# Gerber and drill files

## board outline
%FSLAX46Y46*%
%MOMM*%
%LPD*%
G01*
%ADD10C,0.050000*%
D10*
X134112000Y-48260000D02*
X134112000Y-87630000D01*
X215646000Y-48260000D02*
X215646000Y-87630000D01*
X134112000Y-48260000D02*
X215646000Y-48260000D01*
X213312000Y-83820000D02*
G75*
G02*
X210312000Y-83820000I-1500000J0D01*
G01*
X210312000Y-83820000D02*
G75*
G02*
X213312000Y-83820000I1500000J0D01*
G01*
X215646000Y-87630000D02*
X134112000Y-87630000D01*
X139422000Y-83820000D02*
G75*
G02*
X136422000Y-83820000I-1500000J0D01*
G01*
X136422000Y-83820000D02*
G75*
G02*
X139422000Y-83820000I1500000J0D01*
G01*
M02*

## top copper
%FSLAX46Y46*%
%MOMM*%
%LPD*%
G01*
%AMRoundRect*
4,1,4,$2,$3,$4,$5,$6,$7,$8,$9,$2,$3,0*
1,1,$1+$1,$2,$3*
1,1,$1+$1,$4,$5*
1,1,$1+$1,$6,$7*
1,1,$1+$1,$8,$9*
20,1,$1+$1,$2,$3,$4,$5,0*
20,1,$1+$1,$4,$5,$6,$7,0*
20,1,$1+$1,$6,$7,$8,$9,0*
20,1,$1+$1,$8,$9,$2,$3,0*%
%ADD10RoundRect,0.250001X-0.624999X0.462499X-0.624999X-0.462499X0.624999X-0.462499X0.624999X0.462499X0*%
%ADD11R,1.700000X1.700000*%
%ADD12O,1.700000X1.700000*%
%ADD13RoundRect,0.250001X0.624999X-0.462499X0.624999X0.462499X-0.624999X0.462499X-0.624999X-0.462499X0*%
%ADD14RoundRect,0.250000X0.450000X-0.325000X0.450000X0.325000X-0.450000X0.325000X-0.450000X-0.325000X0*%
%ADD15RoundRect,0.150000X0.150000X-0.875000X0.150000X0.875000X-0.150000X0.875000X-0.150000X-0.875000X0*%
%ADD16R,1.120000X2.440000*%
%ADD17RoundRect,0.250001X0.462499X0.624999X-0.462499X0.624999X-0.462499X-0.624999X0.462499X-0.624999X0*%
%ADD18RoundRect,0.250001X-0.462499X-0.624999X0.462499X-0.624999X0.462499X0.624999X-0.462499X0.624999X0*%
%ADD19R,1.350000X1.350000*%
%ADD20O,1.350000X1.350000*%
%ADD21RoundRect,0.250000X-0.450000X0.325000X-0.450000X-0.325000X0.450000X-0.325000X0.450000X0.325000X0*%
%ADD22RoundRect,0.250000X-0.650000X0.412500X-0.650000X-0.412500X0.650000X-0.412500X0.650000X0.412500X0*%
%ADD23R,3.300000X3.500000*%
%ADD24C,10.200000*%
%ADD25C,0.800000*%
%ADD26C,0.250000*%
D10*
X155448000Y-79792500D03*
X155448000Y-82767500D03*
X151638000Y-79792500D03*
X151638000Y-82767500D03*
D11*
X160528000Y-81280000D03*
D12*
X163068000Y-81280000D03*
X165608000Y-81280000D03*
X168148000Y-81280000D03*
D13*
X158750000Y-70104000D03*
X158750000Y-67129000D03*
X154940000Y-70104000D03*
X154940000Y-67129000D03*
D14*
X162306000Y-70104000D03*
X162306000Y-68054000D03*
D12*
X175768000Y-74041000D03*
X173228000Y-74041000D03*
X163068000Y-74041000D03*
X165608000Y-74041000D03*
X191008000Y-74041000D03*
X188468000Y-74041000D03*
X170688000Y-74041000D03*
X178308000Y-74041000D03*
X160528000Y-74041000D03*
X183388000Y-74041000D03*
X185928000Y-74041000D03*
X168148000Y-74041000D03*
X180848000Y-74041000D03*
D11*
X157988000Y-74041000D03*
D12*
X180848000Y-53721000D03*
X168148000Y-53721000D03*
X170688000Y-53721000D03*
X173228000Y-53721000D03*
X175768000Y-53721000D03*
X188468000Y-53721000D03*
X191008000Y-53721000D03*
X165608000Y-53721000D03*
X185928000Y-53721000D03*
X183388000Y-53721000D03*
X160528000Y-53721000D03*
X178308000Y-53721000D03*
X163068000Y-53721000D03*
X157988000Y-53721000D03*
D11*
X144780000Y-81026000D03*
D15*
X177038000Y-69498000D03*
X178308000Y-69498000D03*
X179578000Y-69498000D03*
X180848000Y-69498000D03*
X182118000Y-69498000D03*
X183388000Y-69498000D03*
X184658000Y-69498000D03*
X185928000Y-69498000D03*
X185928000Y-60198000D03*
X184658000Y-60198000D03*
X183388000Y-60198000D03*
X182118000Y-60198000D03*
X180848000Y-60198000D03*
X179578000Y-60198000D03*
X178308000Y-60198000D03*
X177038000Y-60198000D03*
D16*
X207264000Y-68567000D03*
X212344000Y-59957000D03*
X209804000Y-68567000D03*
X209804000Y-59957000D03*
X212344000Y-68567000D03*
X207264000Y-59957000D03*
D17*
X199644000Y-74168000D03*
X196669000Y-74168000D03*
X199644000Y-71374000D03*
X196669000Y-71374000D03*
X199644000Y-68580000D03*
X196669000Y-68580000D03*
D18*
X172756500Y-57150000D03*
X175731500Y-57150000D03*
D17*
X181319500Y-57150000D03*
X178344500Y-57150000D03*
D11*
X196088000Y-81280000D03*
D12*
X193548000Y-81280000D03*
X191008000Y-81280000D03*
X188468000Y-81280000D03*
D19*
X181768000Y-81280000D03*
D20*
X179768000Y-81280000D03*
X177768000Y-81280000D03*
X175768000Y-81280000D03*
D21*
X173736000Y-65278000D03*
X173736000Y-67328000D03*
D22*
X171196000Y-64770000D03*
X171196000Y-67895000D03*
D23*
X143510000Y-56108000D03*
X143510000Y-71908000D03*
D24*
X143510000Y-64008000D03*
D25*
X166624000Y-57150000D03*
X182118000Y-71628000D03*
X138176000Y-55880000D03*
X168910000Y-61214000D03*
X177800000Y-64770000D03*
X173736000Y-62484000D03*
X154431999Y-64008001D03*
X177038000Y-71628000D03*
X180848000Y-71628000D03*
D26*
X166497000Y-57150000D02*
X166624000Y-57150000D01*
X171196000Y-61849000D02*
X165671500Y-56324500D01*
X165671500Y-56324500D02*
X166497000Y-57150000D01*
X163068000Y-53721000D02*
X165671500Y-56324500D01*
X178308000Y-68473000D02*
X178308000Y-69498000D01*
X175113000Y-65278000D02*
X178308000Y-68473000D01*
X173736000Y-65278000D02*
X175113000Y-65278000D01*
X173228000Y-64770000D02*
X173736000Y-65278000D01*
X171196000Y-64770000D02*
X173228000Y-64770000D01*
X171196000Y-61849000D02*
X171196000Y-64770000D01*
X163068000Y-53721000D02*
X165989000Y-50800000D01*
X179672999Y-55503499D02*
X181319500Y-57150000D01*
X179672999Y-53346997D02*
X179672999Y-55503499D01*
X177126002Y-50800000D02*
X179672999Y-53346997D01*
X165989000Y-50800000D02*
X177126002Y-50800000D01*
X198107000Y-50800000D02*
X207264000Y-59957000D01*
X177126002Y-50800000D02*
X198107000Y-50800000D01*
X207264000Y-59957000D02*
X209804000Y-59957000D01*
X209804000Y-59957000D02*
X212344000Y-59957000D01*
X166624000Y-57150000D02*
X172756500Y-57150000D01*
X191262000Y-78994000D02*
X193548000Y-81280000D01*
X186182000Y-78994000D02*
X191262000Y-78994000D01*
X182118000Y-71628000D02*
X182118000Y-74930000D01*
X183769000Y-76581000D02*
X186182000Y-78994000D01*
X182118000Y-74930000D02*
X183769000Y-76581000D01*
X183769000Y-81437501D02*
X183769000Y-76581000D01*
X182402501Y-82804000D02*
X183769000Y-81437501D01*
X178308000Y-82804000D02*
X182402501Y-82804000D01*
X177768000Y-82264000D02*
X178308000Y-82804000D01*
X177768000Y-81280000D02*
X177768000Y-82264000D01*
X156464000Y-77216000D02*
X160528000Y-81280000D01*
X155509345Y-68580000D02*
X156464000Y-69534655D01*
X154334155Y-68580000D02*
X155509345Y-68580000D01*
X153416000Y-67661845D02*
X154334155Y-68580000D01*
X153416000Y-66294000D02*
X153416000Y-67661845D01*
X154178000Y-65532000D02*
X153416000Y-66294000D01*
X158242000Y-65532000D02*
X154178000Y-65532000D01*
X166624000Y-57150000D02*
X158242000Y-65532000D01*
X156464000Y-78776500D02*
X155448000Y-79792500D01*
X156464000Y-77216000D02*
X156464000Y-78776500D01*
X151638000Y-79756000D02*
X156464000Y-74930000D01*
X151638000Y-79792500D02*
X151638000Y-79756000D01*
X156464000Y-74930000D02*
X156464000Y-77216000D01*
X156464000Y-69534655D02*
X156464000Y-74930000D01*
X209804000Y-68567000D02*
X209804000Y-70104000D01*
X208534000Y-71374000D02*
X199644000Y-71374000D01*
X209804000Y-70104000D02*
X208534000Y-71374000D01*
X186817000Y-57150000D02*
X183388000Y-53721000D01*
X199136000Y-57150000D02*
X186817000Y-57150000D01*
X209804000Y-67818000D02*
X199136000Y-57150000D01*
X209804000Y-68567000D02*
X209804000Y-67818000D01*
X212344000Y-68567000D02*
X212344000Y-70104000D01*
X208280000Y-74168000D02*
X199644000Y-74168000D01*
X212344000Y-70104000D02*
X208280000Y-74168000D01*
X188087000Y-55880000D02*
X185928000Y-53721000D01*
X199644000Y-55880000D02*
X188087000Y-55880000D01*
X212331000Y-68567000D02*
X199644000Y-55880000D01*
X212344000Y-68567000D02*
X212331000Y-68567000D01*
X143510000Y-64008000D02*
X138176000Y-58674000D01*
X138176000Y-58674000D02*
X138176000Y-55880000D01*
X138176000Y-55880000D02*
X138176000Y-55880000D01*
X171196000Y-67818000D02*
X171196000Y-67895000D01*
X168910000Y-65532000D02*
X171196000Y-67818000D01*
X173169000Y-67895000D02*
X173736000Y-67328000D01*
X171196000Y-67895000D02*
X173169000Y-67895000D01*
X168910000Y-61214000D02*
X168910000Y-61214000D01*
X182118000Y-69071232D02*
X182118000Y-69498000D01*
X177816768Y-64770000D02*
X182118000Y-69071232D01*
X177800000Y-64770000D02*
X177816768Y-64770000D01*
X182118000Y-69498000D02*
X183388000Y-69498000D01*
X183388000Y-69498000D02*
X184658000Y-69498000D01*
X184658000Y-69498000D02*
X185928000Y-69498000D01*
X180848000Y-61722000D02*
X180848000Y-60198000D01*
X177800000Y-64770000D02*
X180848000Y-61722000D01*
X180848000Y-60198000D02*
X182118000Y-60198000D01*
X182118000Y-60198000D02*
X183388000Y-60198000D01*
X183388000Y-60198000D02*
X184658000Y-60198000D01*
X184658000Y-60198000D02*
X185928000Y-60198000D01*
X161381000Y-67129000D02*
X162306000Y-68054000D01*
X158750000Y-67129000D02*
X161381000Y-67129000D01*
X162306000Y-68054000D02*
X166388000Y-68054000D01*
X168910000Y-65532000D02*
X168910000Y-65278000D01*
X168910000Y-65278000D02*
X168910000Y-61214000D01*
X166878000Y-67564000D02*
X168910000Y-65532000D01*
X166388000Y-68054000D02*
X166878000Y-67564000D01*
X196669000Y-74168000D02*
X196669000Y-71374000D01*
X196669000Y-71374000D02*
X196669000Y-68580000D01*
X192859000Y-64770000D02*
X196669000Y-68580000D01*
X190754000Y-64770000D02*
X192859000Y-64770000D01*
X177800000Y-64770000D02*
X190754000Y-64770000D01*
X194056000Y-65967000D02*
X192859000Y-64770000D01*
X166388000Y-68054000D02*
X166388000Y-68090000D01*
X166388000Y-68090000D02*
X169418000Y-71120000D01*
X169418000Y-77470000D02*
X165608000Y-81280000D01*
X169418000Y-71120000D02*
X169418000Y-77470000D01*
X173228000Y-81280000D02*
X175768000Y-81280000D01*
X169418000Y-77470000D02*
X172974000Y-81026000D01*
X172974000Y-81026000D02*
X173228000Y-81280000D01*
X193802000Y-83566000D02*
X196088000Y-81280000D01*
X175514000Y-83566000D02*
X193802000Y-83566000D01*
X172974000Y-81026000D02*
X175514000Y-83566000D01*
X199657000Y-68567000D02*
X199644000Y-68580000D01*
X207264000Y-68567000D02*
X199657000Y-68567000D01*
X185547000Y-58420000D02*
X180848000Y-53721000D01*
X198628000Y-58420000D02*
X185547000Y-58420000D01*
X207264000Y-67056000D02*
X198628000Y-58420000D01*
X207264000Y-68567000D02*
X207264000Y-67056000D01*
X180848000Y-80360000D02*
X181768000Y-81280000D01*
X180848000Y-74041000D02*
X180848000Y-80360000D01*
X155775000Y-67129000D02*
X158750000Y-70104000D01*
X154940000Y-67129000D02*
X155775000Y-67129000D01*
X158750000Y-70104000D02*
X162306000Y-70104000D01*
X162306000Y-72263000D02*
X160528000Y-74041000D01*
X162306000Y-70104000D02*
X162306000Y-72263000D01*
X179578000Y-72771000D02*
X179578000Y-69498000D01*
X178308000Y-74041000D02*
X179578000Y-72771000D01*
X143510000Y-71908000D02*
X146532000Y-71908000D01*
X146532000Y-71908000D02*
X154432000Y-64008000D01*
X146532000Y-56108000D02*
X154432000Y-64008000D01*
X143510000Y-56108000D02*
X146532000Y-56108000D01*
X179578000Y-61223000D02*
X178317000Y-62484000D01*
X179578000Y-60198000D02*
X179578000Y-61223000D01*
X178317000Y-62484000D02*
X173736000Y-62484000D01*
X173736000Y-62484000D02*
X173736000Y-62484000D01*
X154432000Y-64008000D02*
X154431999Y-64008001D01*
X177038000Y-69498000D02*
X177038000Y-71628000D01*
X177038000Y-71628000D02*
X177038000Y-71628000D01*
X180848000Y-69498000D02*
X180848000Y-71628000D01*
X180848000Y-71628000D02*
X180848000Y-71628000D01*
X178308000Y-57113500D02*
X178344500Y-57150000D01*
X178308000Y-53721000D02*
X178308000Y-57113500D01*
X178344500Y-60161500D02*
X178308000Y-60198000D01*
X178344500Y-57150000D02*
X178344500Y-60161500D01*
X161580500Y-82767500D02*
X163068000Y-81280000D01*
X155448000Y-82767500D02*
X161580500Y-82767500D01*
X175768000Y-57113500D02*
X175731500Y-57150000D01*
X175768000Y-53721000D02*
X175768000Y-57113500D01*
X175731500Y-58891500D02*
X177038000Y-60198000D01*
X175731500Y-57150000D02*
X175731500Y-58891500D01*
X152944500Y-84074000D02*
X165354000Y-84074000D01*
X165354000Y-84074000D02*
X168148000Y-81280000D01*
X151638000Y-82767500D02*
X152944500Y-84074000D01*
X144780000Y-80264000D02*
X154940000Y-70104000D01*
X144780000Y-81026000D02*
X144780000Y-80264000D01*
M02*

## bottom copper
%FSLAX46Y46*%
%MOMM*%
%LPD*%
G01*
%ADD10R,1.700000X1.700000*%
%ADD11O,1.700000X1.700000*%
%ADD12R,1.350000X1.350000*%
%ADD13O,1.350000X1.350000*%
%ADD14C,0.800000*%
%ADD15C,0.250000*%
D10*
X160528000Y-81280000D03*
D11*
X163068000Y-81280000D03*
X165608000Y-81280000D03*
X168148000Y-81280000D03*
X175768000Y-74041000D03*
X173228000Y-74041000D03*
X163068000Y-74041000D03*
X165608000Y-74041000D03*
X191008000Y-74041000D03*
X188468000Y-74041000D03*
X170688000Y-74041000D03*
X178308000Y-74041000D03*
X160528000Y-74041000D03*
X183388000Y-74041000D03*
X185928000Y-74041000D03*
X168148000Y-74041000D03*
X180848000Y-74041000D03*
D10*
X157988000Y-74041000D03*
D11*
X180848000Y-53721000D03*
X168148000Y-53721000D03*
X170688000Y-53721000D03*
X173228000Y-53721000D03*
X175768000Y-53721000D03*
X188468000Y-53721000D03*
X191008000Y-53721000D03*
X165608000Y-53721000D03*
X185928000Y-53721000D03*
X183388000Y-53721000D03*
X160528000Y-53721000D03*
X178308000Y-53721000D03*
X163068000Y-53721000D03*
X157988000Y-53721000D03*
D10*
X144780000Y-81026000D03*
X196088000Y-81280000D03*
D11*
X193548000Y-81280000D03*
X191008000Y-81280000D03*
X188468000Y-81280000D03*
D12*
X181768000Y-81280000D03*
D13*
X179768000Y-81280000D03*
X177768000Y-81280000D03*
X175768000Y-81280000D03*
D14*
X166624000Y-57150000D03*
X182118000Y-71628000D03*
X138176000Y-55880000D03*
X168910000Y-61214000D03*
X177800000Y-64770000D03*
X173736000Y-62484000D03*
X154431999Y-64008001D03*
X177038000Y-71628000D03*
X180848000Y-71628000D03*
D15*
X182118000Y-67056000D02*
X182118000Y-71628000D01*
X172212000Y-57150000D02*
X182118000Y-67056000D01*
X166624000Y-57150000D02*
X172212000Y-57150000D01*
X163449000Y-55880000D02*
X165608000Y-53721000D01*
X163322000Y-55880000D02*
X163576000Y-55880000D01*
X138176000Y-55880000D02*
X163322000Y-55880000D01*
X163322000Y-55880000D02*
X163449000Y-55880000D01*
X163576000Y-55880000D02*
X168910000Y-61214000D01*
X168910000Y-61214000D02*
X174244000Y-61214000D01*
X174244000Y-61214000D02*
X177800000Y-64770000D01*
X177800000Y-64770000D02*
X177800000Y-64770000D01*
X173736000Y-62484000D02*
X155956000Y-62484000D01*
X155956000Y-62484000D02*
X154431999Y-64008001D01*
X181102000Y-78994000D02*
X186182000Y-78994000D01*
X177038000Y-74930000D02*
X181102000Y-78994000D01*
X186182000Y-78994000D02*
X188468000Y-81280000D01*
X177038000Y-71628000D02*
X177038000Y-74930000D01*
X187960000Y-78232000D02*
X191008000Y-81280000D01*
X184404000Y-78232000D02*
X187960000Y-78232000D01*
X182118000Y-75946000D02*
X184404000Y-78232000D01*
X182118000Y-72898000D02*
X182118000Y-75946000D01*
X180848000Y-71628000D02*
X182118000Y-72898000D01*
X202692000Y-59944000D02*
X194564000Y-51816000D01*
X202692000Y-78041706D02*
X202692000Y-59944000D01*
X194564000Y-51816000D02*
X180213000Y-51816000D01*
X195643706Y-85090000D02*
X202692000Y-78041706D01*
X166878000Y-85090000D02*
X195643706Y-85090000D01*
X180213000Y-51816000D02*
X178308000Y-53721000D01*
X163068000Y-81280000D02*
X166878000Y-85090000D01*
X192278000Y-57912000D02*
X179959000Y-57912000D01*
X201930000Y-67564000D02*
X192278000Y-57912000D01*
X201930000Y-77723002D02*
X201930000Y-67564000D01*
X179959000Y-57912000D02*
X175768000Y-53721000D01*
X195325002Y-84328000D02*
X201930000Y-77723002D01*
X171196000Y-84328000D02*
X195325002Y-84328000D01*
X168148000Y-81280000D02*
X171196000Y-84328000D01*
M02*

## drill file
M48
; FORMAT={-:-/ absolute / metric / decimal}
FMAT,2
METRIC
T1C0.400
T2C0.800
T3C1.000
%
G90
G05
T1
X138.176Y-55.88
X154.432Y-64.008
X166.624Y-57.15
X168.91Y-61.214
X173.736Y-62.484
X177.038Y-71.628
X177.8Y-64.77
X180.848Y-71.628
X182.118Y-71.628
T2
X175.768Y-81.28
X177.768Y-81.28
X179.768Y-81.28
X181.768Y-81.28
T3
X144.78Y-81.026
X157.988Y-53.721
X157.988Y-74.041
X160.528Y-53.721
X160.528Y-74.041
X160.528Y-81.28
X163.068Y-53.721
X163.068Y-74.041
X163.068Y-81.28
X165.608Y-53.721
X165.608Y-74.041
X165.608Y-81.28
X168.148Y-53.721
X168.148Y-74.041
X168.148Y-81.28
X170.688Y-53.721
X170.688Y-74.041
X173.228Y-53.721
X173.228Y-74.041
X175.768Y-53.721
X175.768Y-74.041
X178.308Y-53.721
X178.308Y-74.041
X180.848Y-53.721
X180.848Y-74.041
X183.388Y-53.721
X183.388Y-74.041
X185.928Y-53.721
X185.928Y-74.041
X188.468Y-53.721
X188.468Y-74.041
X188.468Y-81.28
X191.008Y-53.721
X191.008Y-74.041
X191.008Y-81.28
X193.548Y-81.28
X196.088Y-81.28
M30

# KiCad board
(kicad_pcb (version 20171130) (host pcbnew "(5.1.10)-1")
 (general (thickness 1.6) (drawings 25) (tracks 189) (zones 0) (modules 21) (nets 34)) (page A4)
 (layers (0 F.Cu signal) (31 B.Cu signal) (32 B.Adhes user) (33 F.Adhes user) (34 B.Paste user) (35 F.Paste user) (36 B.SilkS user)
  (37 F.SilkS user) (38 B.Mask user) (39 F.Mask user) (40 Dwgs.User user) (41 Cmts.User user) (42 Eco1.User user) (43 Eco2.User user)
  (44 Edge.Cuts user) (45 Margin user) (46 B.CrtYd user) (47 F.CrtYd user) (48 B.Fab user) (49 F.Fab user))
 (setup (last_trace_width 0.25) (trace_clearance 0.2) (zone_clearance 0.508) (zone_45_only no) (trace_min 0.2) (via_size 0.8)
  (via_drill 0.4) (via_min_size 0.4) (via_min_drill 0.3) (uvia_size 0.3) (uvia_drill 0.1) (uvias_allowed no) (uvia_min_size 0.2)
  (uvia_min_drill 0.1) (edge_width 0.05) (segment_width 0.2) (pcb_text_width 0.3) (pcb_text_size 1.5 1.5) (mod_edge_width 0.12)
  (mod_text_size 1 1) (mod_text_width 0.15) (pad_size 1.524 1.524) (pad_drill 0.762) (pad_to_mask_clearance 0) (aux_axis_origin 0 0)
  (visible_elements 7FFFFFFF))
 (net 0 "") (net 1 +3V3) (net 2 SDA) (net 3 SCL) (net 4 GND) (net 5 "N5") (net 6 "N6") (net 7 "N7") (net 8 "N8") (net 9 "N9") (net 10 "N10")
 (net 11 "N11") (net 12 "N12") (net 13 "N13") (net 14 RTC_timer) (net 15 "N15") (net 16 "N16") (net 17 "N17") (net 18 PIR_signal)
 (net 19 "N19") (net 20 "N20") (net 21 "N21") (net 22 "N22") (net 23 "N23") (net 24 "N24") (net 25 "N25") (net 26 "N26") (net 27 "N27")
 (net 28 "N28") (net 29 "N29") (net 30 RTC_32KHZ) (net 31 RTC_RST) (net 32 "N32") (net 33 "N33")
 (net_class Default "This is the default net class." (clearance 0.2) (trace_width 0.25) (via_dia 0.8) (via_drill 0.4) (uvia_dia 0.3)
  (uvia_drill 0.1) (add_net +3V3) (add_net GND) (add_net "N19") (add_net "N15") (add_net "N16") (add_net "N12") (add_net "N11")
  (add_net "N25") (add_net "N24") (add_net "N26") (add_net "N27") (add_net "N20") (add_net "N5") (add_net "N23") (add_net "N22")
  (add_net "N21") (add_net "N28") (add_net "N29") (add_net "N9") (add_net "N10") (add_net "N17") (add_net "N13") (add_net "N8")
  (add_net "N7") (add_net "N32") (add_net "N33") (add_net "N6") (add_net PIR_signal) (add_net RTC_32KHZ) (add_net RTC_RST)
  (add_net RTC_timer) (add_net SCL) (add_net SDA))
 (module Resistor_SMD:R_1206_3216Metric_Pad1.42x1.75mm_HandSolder (layer F.Cu) (at 155.448 81.28 270)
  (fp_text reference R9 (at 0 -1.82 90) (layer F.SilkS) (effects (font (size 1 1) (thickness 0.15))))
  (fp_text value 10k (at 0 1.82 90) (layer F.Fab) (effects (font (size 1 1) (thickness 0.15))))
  (pad 1 smd roundrect (at -1.4875 0 270) (size 1.425 1.75) (layers F.Cu F.Paste F.Mask) (roundrect_rratio 0.175439) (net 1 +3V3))
  (pad 2 smd roundrect (at 1.4875 0 270) (size 1.425 1.75) (layers F.Cu F.Paste F.Mask) (roundrect_rratio 0.175439) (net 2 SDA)))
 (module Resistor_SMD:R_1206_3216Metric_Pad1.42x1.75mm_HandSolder (layer F.Cu) (at 151.638 81.28 270)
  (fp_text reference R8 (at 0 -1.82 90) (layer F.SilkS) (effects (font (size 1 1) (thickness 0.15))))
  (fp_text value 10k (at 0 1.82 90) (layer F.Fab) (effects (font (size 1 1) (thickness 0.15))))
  (pad 1 smd roundrect (at -1.4875 0 270) (size 1.425 1.75) (layers F.Cu F.Paste F.Mask) (roundrect_rratio 0.175439) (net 1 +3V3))
  (pad 2 smd roundrect (at 1.4875 0 270) (size 1.425 1.75) (layers F.Cu F.Paste F.Mask) (roundrect_rratio 0.175439) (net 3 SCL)))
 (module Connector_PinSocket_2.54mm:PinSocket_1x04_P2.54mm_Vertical (layer F.Cu) (at 160.528 81.28 90)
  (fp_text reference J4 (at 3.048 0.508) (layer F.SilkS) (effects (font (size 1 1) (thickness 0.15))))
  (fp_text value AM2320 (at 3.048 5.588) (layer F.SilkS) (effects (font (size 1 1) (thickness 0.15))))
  (pad 1 thru_hole rect (at 0 0 90) (size 1.7 1.7) (drill 1) (layers *.Cu *.Mask) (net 1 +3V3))
  (pad 2 thru_hole oval (at 0 2.54 90) (size 1.7 1.7) (drill 1) (layers *.Cu *.Mask) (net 2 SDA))
  (pad 3 thru_hole oval (at 0 5.08 90) (size 1.7 1.7) (drill 1) (layers *.Cu *.Mask) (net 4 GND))
  (pad 4 thru_hole oval (at 0 7.62 90) (size 1.7 1.7) (drill 1) (layers *.Cu *.Mask) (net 3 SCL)))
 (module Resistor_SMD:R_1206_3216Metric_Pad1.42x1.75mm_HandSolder (layer F.Cu) (at 158.75 68.6165 90)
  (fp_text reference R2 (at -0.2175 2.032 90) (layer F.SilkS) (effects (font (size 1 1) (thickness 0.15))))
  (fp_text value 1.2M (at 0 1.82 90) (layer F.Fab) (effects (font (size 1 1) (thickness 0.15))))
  (pad 1 smd roundrect (at -1.4875 0 90) (size 1.425 1.75) (layers F.Cu F.Paste F.Mask) (roundrect_rratio 0.175439) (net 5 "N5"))
  (pad 2 smd roundrect (at 1.4875 0 90) (size 1.425 1.75) (layers F.Cu F.Paste F.Mask) (roundrect_rratio 0.175439) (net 4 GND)))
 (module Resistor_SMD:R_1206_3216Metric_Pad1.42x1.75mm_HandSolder (layer F.Cu) (at 154.94 68.6165 90)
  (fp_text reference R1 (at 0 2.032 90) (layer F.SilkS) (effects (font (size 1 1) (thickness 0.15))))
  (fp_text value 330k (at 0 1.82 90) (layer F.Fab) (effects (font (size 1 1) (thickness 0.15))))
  (pad 1 smd roundrect (at -1.4875 0 90) (size 1.425 1.75) (layers F.Cu F.Paste F.Mask) (roundrect_rratio 0.175439) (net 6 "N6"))
  (pad 2 smd roundrect (at 1.4875 0 90) (size 1.425 1.75) (layers F.Cu F.Paste F.Mask) (roundrect_rratio 0.175439) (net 5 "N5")))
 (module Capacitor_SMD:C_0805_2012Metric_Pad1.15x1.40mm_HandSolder (layer F.Cu) (at 162.306 69.079 90)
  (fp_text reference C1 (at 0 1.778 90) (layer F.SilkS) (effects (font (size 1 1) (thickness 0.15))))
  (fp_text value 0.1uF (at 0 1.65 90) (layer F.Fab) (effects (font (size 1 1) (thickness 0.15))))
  (pad 1 smd roundrect (at -1.025 0 90) (size 1.15 1.4) (layers F.Cu F.Paste F.Mask) (roundrect_rratio 0.217391) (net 5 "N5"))
  (pad 2 smd roundrect (at 1.025 0 90) (size 1.15 1.4) (layers F.Cu F.Paste F.Mask) (roundrect_rratio 0.217391) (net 4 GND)))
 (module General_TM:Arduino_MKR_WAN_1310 (layer F.Cu) (at 157.988 74.041 90)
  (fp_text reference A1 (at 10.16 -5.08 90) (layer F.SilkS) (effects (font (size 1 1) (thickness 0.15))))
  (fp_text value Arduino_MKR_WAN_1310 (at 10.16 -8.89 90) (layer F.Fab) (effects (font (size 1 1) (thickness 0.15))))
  (pad 8 thru_hole oval (at 0 17.78 90) (size 1.7 1.7) (drill 1) (layers *.Cu *.Mask) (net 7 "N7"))
  (pad 7 thru_hole oval (at 0 15.24 90) (size 1.7 1.7) (drill 1) (layers *.Cu *.Mask) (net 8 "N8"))
  (pad 3 thru_hole oval (at 0 5.08 90) (size 1.7 1.7) (drill 1) (layers *.Cu *.Mask) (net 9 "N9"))
  (pad 4 thru_hole oval (at 0 7.62 90) (size 1.7 1.7) (drill 1) (layers *.Cu *.Mask) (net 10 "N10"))
  (pad 14 thru_hole oval (at 0 33.02 90) (size 1.7 1.7) (drill 1) (layers *.Cu *.Mask) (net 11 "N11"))
  (pad 13 thru_hole oval (at 0 30.48 90) (size 1.7 1.7) (drill 1) (layers *.Cu *.Mask) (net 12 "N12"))
  (pad 6 thru_hole oval (at 0 12.7 90) (size 1.7 1.7) (drill 1) (layers *.Cu *.Mask) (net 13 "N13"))
  (pad 9 thru_hole oval (at 0 20.32 90) (size 1.7 1.7) (drill 1) (layers *.Cu *.Mask) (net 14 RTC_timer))
  (pad 2 thru_hole oval (at 0 2.54 90) (size 1.7 1.7) (drill 1) (layers *.Cu *.Mask) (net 5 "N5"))
  (pad 11 thru_hole oval (at 0 25.4 90) (size 1.7 1.7) (drill 1) (layers *.Cu *.Mask) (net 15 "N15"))
  (pad 12 thru_hole oval (at 0 27.94 90) (size 1.7 1.7) (drill 1) (layers *.Cu *.Mask) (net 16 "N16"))
  (pad 5 thru_hole oval (at 0 10.16 90) (size 1.7 1.7) (drill 1) (layers *.Cu *.Mask) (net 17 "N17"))
  (pad 10 thru_hole oval (at 0 22.86 90) (size 1.7 1.7) (drill 1) (layers *.Cu *.Mask) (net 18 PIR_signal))
  (pad 1 thru_hole rect (at 0 0 90) (size 1.7 1.7) (drill 1) (layers *.Cu *.Mask) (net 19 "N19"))
  (pad 19 thru_hole oval (at 20.32 22.86 90) (size 1.7 1.7) (drill 1) (layers *.Cu *.Mask) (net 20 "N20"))
  (pad 24 thru_hole oval (at 20.32 10.16 90) (size 1.7 1.7) (drill 1) (layers *.Cu *.Mask) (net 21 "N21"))
  (pad 23 thru_hole oval (at 20.32 12.7 90) (size 1.7 1.7) (drill 1) (layers *.Cu *.Mask) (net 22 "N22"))
  (pad 22 thru_hole oval (at 20.32 15.24 90) (size 1.7 1.7) (drill 1) (layers *.Cu *.Mask) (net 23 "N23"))
  (pad 21 thru_hole oval (at 20.32 17.78 90) (size 1.7 1.7) (drill 1) (layers *.Cu *.Mask) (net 3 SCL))
  (pad 16 thru_hole oval (at 20.32 30.48 90) (size 1.7 1.7) (drill 1) (layers *.Cu *.Mask) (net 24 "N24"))
  (pad 15 thru_hole oval (at 20.32 33.02 90) (size 1.7 1.7) (drill 1) (layers *.Cu *.Mask) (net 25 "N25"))
  (pad 25 thru_hole oval (at 20.32 7.62 90) (size 1.7 1.7) (drill 1) (layers *.Cu *.Mask) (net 4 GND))
  (pad 17 thru_hole oval (at 20.32 27.94 90) (size 1.7 1.7) (drill 1) (layers *.Cu *.Mask) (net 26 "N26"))
  (pad 18 thru_hole oval (at 20.32 25.4 90) (size 1.7 1.7) (drill 1) (layers *.Cu *.Mask) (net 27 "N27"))
  (pad 27 thru_hole oval (at 20.32 2.54 90) (size 1.7 1.7) (drill 1) (layers *.Cu *.Mask) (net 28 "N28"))
  (pad 20 thru_hole oval (at 20.32 20.32 90) (size 1.7 1.7) (drill 1) (layers *.Cu *.Mask) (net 2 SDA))
  (pad 26 thru_hole oval (at 20.32 5.08 90) (size 1.7 1.7) (drill 1) (layers *.Cu *.Mask) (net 1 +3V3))
  (pad 28 thru_hole oval (at 20.32 0 90) (size 1.7 1.7) (drill 1) (layers *.Cu *.Mask) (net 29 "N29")))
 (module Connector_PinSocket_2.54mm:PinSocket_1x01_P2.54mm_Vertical (layer F.Cu) (at 144.78 81.026)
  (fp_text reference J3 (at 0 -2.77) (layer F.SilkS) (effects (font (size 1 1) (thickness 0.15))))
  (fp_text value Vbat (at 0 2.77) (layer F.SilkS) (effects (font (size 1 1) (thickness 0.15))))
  (pad 1 thru_hole rect (at 0 0) (size 1.7 1.7) (drill 1) (layers *.Cu *.Mask) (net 6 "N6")))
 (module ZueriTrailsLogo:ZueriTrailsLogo (layer B.Cu) (at 173.99 63.754 180)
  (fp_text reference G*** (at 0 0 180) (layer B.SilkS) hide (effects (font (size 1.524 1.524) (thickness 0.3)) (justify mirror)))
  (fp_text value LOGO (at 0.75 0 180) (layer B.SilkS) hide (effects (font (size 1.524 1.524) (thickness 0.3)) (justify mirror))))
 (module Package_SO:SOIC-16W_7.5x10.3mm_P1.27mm (layer F.Cu) (at 181.483 64.848 90)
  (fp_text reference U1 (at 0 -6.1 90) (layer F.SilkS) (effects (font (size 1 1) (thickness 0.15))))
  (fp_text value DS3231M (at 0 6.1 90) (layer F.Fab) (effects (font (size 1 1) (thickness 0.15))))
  (pad 1 smd roundrect (at -4.65 -4.445 90) (size 2.05 0.6) (layers F.Cu F.Paste F.Mask) (roundrect_rratio 0.25) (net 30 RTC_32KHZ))
  (pad 2 smd roundrect (at -4.65 -3.175 90) (size 2.05 0.6) (layers F.Cu F.Paste F.Mask) (roundrect_rratio 0.25) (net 1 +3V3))
  (pad 3 smd roundrect (at -4.65 -1.905 90) (size 2.05 0.6) (layers F.Cu F.Paste F.Mask) (roundrect_rratio 0.25) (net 14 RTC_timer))
  (pad 4 smd roundrect (at -4.65 -0.635 90) (size 2.05 0.6) (layers F.Cu F.Paste F.Mask) (roundrect_rratio 0.25) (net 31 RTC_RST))
  (pad 5 smd roundrect (at -4.65 0.635 90) (size 2.05 0.6) (layers F.Cu F.Paste F.Mask) (roundrect_rratio 0.25) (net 4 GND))
  (pad 6 smd roundrect (at -4.65 1.905 90) (size 2.05 0.6) (layers F.Cu F.Paste F.Mask) (roundrect_rratio 0.25) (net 4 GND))
  (pad 7 smd roundrect (at -4.65 3.175 90) (size 2.05 0.6) (layers F.Cu F.Paste F.Mask) (roundrect_rratio 0.25) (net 4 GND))
  (pad 8 smd roundrect (at -4.65 4.445 90) (size 2.05 0.6) (layers F.Cu F.Paste F.Mask) (roundrect_rratio 0.25) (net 4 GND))
  (pad 9 smd roundrect (at 4.65 4.445 90) (size 2.05 0.6) (layers F.Cu F.Paste F.Mask) (roundrect_rratio 0.25) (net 4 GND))
  (pad 10 smd roundrect (at 4.65 3.175 90) (size 2.05 0.6) (layers F.Cu F.Paste F.Mask) (roundrect_rratio 0.25) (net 4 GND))
  (pad 11 smd roundrect (at 4.65 1.905 90) (size 2.05 0.6) (layers F.Cu F.Paste F.Mask) (roundrect_rratio 0.25) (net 4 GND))
  (pad 12 smd roundrect (at 4.65 0.635 90) (size 2.05 0.6) (layers F.Cu F.Paste F.Mask) (roundrect_rratio 0.25) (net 4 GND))
  (pad 13 smd roundrect (at 4.65 -0.635 90) (size 2.05 0.6) (layers F.Cu F.Paste F.Mask) (roundrect_rratio 0.25) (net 4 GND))
  (pad 14 smd roundrect (at 4.65 -1.905 90) (size 2.05 0.6) (layers F.Cu F.Paste F.Mask) (roundrect_rratio 0.25) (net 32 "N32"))
  (pad 15 smd roundrect (at 4.65 -3.175 90) (size 2.05 0.6) (layers F.Cu F.Paste F.Mask) (roundrect_rratio 0.25) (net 2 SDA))
  (pad 16 smd roundrect (at 4.65 -4.445 90) (size 2.05 0.6) (layers F.Cu F.Paste F.Mask) (roundrect_rratio 0.25) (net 3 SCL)))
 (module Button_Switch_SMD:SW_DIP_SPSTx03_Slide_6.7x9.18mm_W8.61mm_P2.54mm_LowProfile (layer F.Cu) (at 209.804 64.262 90)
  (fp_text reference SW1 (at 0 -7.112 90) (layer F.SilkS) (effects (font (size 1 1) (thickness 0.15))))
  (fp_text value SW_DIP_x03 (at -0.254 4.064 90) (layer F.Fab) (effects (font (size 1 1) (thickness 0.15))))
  (pad 1 smd rect (at -4.305 -2.54 90) (size 2.44 1.12) (layers F.Cu F.Paste F.Mask) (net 20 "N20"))
  (pad 4 smd rect (at 4.305 2.54 90) (size 2.44 1.12) (layers F.Cu F.Paste F.Mask) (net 1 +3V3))
  (pad 2 smd rect (at -4.305 0 90) (size 2.44 1.12) (layers F.Cu F.Paste F.Mask) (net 27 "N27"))
  (pad 5 smd rect (at 4.305 0 90) (size 2.44 1.12) (layers F.Cu F.Paste F.Mask) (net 1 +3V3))
  (pad 3 smd rect (at -4.305 2.54 90) (size 2.44 1.12) (layers F.Cu F.Paste F.Mask) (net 26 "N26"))
  (pad 6 smd rect (at 4.305 -2.54 90) (size 2.44 1.12) (layers F.Cu F.Paste F.Mask) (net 1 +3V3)))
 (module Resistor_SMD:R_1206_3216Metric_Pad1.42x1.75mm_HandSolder (layer F.Cu) (at 198.1565 74.168 180)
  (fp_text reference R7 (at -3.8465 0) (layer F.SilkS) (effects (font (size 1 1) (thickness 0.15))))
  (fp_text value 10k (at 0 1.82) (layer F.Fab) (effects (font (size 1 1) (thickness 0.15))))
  (pad 1 smd roundrect (at -1.4875 0 180) (size 1.425 1.75) (layers F.Cu F.Paste F.Mask) (roundrect_rratio 0.175439) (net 26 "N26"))
  (pad 2 smd roundrect (at 1.4875 0 180) (size 1.425 1.75) (layers F.Cu F.Paste F.Mask) (roundrect_rratio 0.175439) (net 4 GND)))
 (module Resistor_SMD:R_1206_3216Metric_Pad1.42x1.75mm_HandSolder (layer F.Cu) (at 198.1565 71.374 180)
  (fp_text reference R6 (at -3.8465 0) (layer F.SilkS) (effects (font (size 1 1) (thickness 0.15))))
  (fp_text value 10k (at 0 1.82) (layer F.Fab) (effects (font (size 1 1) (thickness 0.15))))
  (pad 1 smd roundrect (at -1.4875 0 180) (size 1.425 1.75) (layers F.Cu F.Paste F.Mask) (roundrect_rratio 0.175439) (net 27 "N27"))
  (pad 2 smd roundrect (at 1.4875 0 180) (size 1.425 1.75) (layers F.Cu F.Paste F.Mask) (roundrect_rratio 0.175439) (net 4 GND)))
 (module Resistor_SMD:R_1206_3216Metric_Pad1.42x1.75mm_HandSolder (layer F.Cu) (at 198.1565 68.58 180)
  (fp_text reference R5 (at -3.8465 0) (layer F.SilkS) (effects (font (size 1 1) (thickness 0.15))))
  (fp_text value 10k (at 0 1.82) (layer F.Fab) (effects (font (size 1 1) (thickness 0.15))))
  (pad 1 smd roundrect (at -1.4875 0 180) (size 1.425 1.75) (layers F.Cu F.Paste F.Mask) (roundrect_rratio 0.175439) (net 20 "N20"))
  (pad 2 smd roundrect (at 1.4875 0 180) (size 1.425 1.75) (layers F.Cu F.Paste F.Mask) (roundrect_rratio 0.175439) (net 4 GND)))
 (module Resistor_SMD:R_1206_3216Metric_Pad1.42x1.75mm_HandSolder (layer F.Cu) (at 174.244 57.15)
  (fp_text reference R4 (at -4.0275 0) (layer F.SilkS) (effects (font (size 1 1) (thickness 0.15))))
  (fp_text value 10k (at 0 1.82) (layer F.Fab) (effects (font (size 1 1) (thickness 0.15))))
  (pad 1 smd roundrect (at -1.4875 0) (size 1.425 1.75) (layers F.Cu F.Paste F.Mask) (roundrect_rratio 0.175439) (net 1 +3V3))
  (pad 2 smd roundrect (at 1.4875 0) (size 1.425 1.75) (layers F.Cu F.Paste F.Mask) (roundrect_rratio 0.175439) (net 3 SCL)))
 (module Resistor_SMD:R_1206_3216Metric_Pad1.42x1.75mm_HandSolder (layer F.Cu) (at 179.832 57.15 180)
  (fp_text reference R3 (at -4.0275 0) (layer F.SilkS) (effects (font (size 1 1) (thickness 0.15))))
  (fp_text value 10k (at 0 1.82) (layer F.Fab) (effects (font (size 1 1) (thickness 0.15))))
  (pad 1 smd roundrect (at -1.4875 0 180) (size 1.425 1.75) (layers F.Cu F.Paste F.Mask) (roundrect_rratio 0.175439) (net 1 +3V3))
  (pad 2 smd roundrect (at 1.4875 0 180) (size 1.425 1.75) (layers F.Cu F.Paste F.Mask) (roundrect_rratio 0.175439) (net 2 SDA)))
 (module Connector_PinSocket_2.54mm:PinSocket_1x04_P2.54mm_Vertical (layer F.Cu) (at 196.088 81.28 270)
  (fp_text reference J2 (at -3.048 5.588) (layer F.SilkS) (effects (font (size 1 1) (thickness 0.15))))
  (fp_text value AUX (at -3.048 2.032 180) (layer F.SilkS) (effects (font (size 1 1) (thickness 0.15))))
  (pad 1 thru_hole rect (at 0 0 270) (size 1.7 1.7) (drill 1) (layers *.Cu *.Mask) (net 4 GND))
  (pad 2 thru_hole oval (at 0 2.54 270) (size 1.7 1.7) (drill 1) (layers *.Cu *.Mask) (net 1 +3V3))
  (pad 3 thru_hole oval (at 0 5.08 270) (size 1.7 1.7) (drill 1) (layers *.Cu *.Mask) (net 31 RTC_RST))
  (pad 4 thru_hole oval (at 0 7.62 270) (size 1.7 1.7) (drill 1) (layers *.Cu *.Mask) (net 30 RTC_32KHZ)))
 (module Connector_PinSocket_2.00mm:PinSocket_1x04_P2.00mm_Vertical (layer F.Cu) (at 181.768 81.28 270)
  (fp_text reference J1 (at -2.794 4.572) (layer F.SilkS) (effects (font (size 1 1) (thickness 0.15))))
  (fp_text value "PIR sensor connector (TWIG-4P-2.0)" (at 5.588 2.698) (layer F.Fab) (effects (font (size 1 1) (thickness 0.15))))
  (pad 1 thru_hole rect (at 0 0 270) (size 1.35 1.35) (drill 0.8) (layers *.Cu *.Mask) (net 18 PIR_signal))
  (pad 2 thru_hole oval (at 0 2 270) (size 1.35 1.35) (drill 0.8) (layers *.Cu *.Mask) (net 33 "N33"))
  (pad 3 thru_hole oval (at 0 4 270) (size 1.35 1.35) (drill 0.8) (layers *.Cu *.Mask) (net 1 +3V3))
  (pad 4 thru_hole oval (at 0 6 270) (size 1.35 1.35) (drill 0.8) (layers *.Cu *.Mask) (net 4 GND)))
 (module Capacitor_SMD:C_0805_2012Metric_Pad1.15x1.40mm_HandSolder (layer F.Cu) (at 173.736 66.303 270)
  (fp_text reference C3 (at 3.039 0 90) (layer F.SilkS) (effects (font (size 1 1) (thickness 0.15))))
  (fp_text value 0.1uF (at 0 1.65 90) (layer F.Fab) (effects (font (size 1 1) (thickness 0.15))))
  (pad 1 smd roundrect (at -1.025 0 270) (size 1.15 1.4) (layers F.Cu F.Paste F.Mask) (roundrect_rratio 0.217391) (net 1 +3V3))
  (pad 2 smd roundrect (at 1.025 0 270) (size 1.15 1.4) (layers F.Cu F.Paste F.Mask) (roundrect_rratio 0.217391) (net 4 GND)))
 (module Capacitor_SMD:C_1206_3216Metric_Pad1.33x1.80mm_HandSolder (layer F.Cu) (at 171.196 66.3325 270)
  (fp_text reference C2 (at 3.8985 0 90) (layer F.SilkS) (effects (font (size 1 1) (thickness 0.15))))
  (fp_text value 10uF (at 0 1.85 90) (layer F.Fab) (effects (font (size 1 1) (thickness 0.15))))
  (pad 1 smd roundrect (at -1.5625 0 270) (size 1.325 1.8) (layers F.Cu F.Paste F.Mask) (roundrect_rratio 0.188679) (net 1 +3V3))
  (pad 2 smd roundrect (at 1.5625 0 270) (size 1.325 1.8) (layers F.Cu F.Paste F.Mask) (roundrect_rratio 0.188679) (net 4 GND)))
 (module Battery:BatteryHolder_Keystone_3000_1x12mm (layer F.Cu) (at 143.51 64.008 270)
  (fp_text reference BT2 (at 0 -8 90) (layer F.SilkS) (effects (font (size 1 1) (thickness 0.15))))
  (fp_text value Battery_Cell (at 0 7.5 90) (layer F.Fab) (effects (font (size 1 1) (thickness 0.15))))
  (pad 1 smd rect (at -7.9 0 270) (size 3.5 3.3) (layers F.Cu F.Paste F.Mask) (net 32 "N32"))
  (pad 1 smd rect (at 7.9 0 270) (size 3.5 3.3) (layers F.Cu F.Paste F.Mask) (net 32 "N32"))
  (pad 2 smd circle (at 0 0 270) (size 10.2 10.2) (layers F.Cu F.Mask) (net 4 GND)))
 (gr_line (start 134.112 48.26) (end 134.112 87.63) (layer Edge.Cuts) (width 0.05))
 (gr_line (start 215.646 48.26) (end 215.646 87.63) (layer Edge.Cuts) (width 0.05))
 (gr_line (start 134.112 48.26) (end 215.646 48.26) (layer Edge.Cuts) (width 0.05))
 (gr_circle (center 211.812 83.82) (end 210.312 83.82) (layer Edge.Cuts) (width 0.05))
 (gr_line (start 215.646 87.63) (end 134.112 87.63) (layer Edge.Cuts) (width 0.05))
 (gr_circle (center 137.922 83.82) (end 136.422 83.82) (layer Edge.Cuts) (width 0.05))
 (segment (start 166.497 57.15) (end 166.624 57.15) (width 0.25) (layer F.Cu) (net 1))
 (segment (start 171.196 61.849) (end 165.6715 56.3245) (width 0.25) (layer F.Cu) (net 1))
 (segment (start 165.6715 56.3245) (end 166.497 57.15) (width 0.25) (layer F.Cu) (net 1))
 (segment (start 163.068 53.721) (end 165.6715 56.3245) (width 0.25) (layer F.Cu) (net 1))
 (segment (start 178.308 68.473) (end 178.308 69.498) (width 0.25) (layer F.Cu) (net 1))
 (segment (start 175.113 65.278) (end 178.308 68.473) (width 0.25) (layer F.Cu) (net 1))
 (segment (start 173.736 65.278) (end 175.113 65.278) (width 0.25) (layer F.Cu) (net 1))
 (segment (start 173.228 64.77) (end 173.736 65.278) (width 0.25) (layer F.Cu) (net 1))
 (segment (start 171.196 64.77) (end 173.228 64.77) (width 0.25) (layer F.Cu) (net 1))
 (segment (start 171.196 61.849) (end 171.196 64.77) (width 0.25) (layer F.Cu) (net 1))
 (segment (start 163.068 53.721) (end 165.989 50.8) (width 0.25) (layer F.Cu) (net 1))
 (segment (start 179.672999 55.503499) (end 181.3195 57.15) (width 0.25) (layer F.Cu) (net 1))
 (segment (start 179.672999 53.346997) (end 179.672999 55.503499) (width 0.25) (layer F.Cu) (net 1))
 (segment (start 177.126002 50.8) (end 179.672999 53.346997) (width 0.25) (layer F.Cu) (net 1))
 (segment (start 165.989 50.8) (end 177.126002 50.8) (width 0.25) (layer F.Cu) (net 1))
 (segment (start 198.107 50.8) (end 207.264 59.957) (width 0.25) (layer F.Cu) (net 1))
 (segment (start 177.126002 50.8) (end 198.107 50.8) (width 0.25) (layer F.Cu) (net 1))
 (segment (start 207.264 59.957) (end 209.804 59.957) (width 0.25) (layer F.Cu) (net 1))
 (segment (start 209.804 59.957) (end 212.344 59.957) (width 0.25) (layer F.Cu) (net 1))
 (segment (start 166.624 57.15) (end 172.7565 57.15) (width 0.25) (layer F.Cu) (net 1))
 (via (at 166.624 57.15) (size 0.8) (drill 0.4) (layers F.Cu B.Cu) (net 1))
 (segment (start 182.118 67.056) (end 182.118 71.628) (width 0.25) (layer B.Cu) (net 1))
 (segment (start 172.212 57.15) (end 182.118 67.056) (width 0.25) (layer B.Cu) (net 1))
 (segment (start 166.624 57.15) (end 172.212 57.15) (width 0.25) (layer B.Cu) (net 1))
 (via (at 182.118 71.628) (size 0.8) (drill 0.4) (layers F.Cu B.Cu) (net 1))
 (segment (start 191.262 78.994) (end 193.548 81.28) (width 0.25) (layer F.Cu) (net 1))
 (segment (start 186.182 78.994) (end 191.262 78.994) (width 0.25) (layer F.Cu) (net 1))
 (segment (start 182.118 71.628) (end 182.118 74.93) (width 0.25) (layer F.Cu) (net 1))
 (segment (start 183.769 76.581) (end 186.182 78.994) (width 0.25) (layer F.Cu) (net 1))
 (segment (start 182.118 74.93) (end 183.769 76.581) (width 0.25) (layer F.Cu) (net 1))
 (segment (start 183.769 81.437501) (end 183.769 76.581) (width 0.25) (layer F.Cu) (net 1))
 (segment (start 182.402501 82.804) (end 183.769 81.437501) (width 0.25) (layer F.Cu) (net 1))
 (segment (start 178.308 82.804) (end 182.402501 82.804) (width 0.25) (layer F.Cu) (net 1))
 (segment (start 177.768 82.264) (end 178.308 82.804) (width 0.25) (layer F.Cu) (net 1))
 (segment (start 177.768 81.28) (end 177.768 82.264) (width 0.25) (layer F.Cu) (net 1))
 (segment (start 156.464 77.216) (end 160.528 81.28) (width 0.25) (layer F.Cu) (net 1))
 (segment (start 155.509345 68.58) (end 156.464 69.534655) (width 0.25) (layer F.Cu) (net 1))
 (segment (start 154.334155 68.58) (end 155.509345 68.58) (width 0.25) (layer F.Cu) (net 1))
 (segment (start 153.416 67.661845) (end 154.334155 68.58) (width 0.25) (layer F.Cu) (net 1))
 (segment (start 153.416 66.294) (end 153.416 67.661845) (width 0.25) (layer F.Cu) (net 1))
 (segment (start 154.178 65.532) (end 153.416 66.294) (width 0.25) (layer F.Cu) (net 1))
 (segment (start 158.242 65.532) (end 154.178 65.532) (width 0.25) (layer F.Cu) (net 1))
 (segment (start 166.624 57.15) (end 158.242 65.532) (width 0.25) (layer F.Cu) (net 1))
 (segment (start 156.464 78.7765) (end 155.448 79.7925) (width 0.25) (layer F.Cu) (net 1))
 (segment (start 156.464 77.216) (end 156.464 78.7765) (width 0.25) (layer F.Cu) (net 1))
 (segment (start 151.638 79.756) (end 156.464 74.93) (width 0.25) (layer F.Cu) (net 1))
 (segment (start 151.638 79.7925) (end 151.638 79.756) (width 0.25) (layer F.Cu) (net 1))
 (segment (start 156.464 74.93) (end 156.464 77.216) (width 0.25) (layer F.Cu) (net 1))
 (segment (start 156.464 69.534655) (end 156.464 74.93) (width 0.25) (layer F.Cu) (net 1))
 (segment (start 209.804 68.567) (end 209.804 70.104) (width 0.25) (layer F.Cu) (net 27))
 (segment (start 208.534 71.374) (end 199.644 71.374) (width 0.25) (layer F.Cu) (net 27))
 (segment (start 209.804 70.104) (end 208.534 71.374) (width 0.25) (layer F.Cu) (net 27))
 (segment (start 186.817 57.15) (end 183.388 53.721) (width 0.25) (layer F.Cu) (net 27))
 (segment (start 199.136 57.15) (end 186.817 57.15) (width 0.25) (layer F.Cu) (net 27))
 (segment (start 209.804 67.818) (end 199.136 57.15) (width 0.25) (layer F.Cu) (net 27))
 (segment (start 209.804 68.567) (end 209.804 67.818) (width 0.25) (layer F.Cu) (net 27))
 (segment (start 212.344 68.567) (end 212.344 70.104) (width 0.25) (layer F.Cu) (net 26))
 (segment (start 208.28 74.168) (end 199.644 74.168) (width 0.25) (layer F.Cu) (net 26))
 (segment (start 212.344 70.104) (end 208.28 74.168) (width 0.25) (layer F.Cu) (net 26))
 (segment (start 188.087 55.88) (end 185.928 53.721) (width 0.25) (layer F.Cu) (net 26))
 (segment (start 199.644 55.88) (end 188.087 55.88) (width 0.25) (layer F.Cu) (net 26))
 (segment (start 212.331 68.567) (end 199.644 55.88) (width 0.25) (layer F.Cu) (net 26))
 (segment (start 212.344 68.567) (end 212.331 68.567) (width 0.25) (layer F.Cu) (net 26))
 (segment (start 143.51 64.008) (end 138.176 58.674) (width 0.25) (layer F.Cu) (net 4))
 (segment (start 138.176 58.674) (end 138.176 55.88) (width 0.25) (layer F.Cu) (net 4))
 (segment (start 138.176 55.88) (end 138.176 55.88) (width 0.25) (layer F.Cu) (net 4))
 (via (at 138.176 55.88) (size 0.8) (drill 0.4) (layers F.Cu B.Cu) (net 4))
 (segment (start 163.449 55.88) (end 165.608 53.721) (width 0.25) (layer B.Cu) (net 4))
 (segment (start 163.322 55.88) (end 163.576 55.88) (width 0.25) (layer B.Cu) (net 4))
 (segment (start 138.176 55.88) (end 163.322 55.88) (width 0.25) (layer B.Cu) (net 4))
 (segment (start 163.322 55.88) (end 163.449 55.88) (width 0.25) (layer B.Cu) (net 4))
 (segment (start 163.576 55.88) (end 168.91 61.214) (width 0.25) (layer B.Cu) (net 4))
 (segment (start 171.196 67.818) (end 171.196 67.895) (width 0.25) (layer F.Cu) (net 4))
 (segment (start 168.91 65.532) (end 171.196 67.818) (width 0.25) (layer F.Cu) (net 4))
 (segment (start 173.169 67.895) (end 173.736 67.328) (width 0.25) (layer F.Cu) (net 4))
 (segment (start 171.196 67.895) (end 173.169 67.895) (width 0.25) (layer F.Cu) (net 4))
 (segment (start 168.91 61.214) (end 168.91 61.214) (width 0.25) (layer F.Cu) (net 4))
 (via (at 168.91 61.214) (size 0.8) (drill 0.4) (layers F.Cu B.Cu) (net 4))
 (segment (start 168.91 61.214) (end 174.244 61.214) (width 0.25) (layer B.Cu) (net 4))
 (segment (start 174.244 61.214) (end 177.8 64.77) (width 0.25) (layer B.Cu) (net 4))
 (segment (start 177.8 64.77) (end 177.8 64.77) (width 0.25) (layer B.Cu) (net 4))
 (via (at 177.8 64.77) (size 0.8) (drill 0.4) (layers F.Cu B.Cu) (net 4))
 (segment (start 182.118 69.071232) (end 182.118 69.498) (width 0.25) (layer F.Cu) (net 4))
 (segment (start 177.816768 64.77) (end 182.118 69.071232) (width 0.25) (layer F.Cu) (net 4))
 (segment (start 177.8 64.77) (end 177.816768 64.77) (width 0.25) (layer F.Cu) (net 4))
 (segment (start 182.118 69.498) (end 183.388 69.498) (width 0.25) (layer F.Cu) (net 4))
 (segment (start 183.388 69.498) (end 184.658 69.498) (width 0.25) (layer F.Cu) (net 4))
 (segment (start 184.658 69.498) (end 185.928 69.498) (width 0.25) (layer F.Cu) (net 4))
 (segment (start 180.848 61.722) (end 180.848 60.198) (width 0.25) (layer F.Cu) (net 4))
 (segment (start 177.8 64.77) (end 180.848 61.722) (width 0.25) (layer F.Cu) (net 4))
 (segment (start 180.848 60.198) (end 182.118 60.198) (width 0.25) (layer F.Cu) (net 4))
 (segment (start 182.118 60.198) (end 183.388 60.198) (width 0.25) (layer F.Cu) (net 4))
 (segment (start 183.388 60.198) (end 184.658 60.198) (width 0.25) (layer F.Cu) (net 4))
 (segment (start 184.658 60.198) (end 185.928 60.198) (width 0.25) (layer F.Cu) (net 4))
 (segment (start 161.381 67.129) (end 162.306 68.054) (width 0.25) (layer F.Cu) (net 4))
 (segment (start 158.75 67.129) (end 161.381 67.129) (width 0.25) (layer F.Cu) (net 4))
 (segment (start 162.306 68.054) (end 166.388 68.054) (width 0.25) (layer F.Cu) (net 4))
 (segment (start 168.91 65.532) (end 168.91 65.278) (width 0.25) (layer F.Cu) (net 4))
 (segment (start 168.91 65.278) (end 168.91 61.214) (width 0.25) (layer F.Cu) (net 4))
 (segment (start 166.878 67.564) (end 168.91 65.532) (width 0.25) (layer F.Cu) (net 4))
 (segment (start 166.388 68.054) (end 166.878 67.564) (width 0.25) (layer F.Cu) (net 4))
 (segment (start 196.669 74.168) (end 196.669 71.374) (width 0.25) (layer F.Cu) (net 4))
 (segment (start 196.669 71.374) (end 196.669 68.58) (width 0.25) (layer F.Cu) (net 4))
 (segment (start 192.859 64.77) (end 196.669 68.58) (width 0.25) (layer F.Cu) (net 4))
 (segment (start 190.754 64.77) (end 192.859 64.77) (width 0.25) (layer F.Cu) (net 4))
 (segment (start 177.8 64.77) (end 190.754 64.77) (width 0.25) (layer F.Cu) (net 4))
 (segment (start 194.056 65.967) (end 192.859 64.77) (width 0.25) (layer F.Cu) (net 4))
 (segment (start 166.388 68.054) (end 166.388 68.09) (width 0.25) (layer F.Cu) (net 4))
 (segment (start 166.388 68.09) (end 169.418 71.12) (width 0.25) (layer F.Cu) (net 4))
 (segment (start 169.418 77.47) (end 165.608 81.28) (width 0.25) (layer F.Cu) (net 4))
 (segment (start 169.418 71.12) (end 169.418 77.47) (width 0.25) (layer F.Cu) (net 4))
 (segment (start 173.228 81.28) (end 175.768 81.28) (width 0.25) (layer F.Cu) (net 4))
 (segment (start 169.418 77.47) (end 172.974 81.026) (width 0.25) (layer F.Cu) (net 4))
 (segment (start 172.974 81.026) (end 173.228 81.28) (width 0.25) (layer F.Cu) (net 4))
 (segment (start 193.802 83.566) (end 196.088 81.28) (width 0.25) (layer F.Cu) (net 4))
 (segment (start 175.514 83.566) (end 193.802 83.566) (width 0.25) (layer F.Cu) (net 4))
 (segment (start 172.974 81.026) (end 175.514 83.566) (width 0.25) (layer F.Cu) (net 4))
 (segment (start 199.657 68.567) (end 199.644 68.58) (width 0.25) (layer F.Cu) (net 20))
 (segment (start 207.264 68.567) (end 199.657 68.567) (width 0.25) (layer F.Cu) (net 20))
 (segment (start 185.547 58.42) (end 180.848 53.721) (width 0.25) (layer F.Cu) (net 20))
 (segment (start 198.628 58.42) (end 185.547 58.42) (width 0.25) (layer F.Cu) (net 20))
 (segment (start 207.264 67.056) (end 198.628 58.42) (width 0.25) (layer F.Cu) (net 20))
 (segment (start 207.264 68.567) (end 207.264 67.056) (width 0.25) (layer F.Cu) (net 20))
 (segment (start 180.848 80.36) (end 181.768 81.28) (width 0.25) (layer F.Cu) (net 18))
 (segment (start 180.848 74.041) (end 180.848 80.36) (width 0.25) (layer F.Cu) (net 18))
 (segment (start 155.775 67.129) (end 158.75 70.104) (width 0.25) (layer F.Cu) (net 5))
 (segment (start 154.94 67.129) (end 155.775 67.129) (width 0.25) (layer F.Cu) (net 5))
 (segment (start 158.75 70.104) (end 162.306 70.104) (width 0.25) (layer F.Cu) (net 5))
 (segment (start 162.306 72.263) (end 160.528 74.041) (width 0.25) (layer F.Cu) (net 5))
 (segment (start 162.306 70.104) (end 162.306 72.263) (width 0.25) (layer F.Cu) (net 5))
 (segment (start 179.578 72.771) (end 179.578 69.498) (width 0.25) (layer F.Cu) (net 14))
 (segment (start 178.308 74.041) (end 179.578 72.771) (width 0.25) (layer F.Cu) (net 14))
 (segment (start 143.51 71.908) (end 146.532 71.908) (width 0.25) (layer F.Cu) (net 32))
 (segment (start 146.532 71.908) (end 154.432 64.008) (width 0.25) (layer F.Cu) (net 32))
 (segment (start 146.532 56.108) (end 154.432 64.008) (width 0.25) (layer F.Cu) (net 32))
 (segment (start 143.51 56.108) (end 146.532 56.108) (width 0.25) (layer F.Cu) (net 32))
 (segment (start 179.578 61.223) (end 178.317 62.484) (width 0.25) (layer F.Cu) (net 32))
 (segment (start 179.578 60.198) (end 179.578 61.223) (width 0.25) (layer F.Cu) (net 32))
 (segment (start 178.317 62.484) (end 173.736 62.484) (width 0.25) (layer F.Cu) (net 32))
 (segment (start 173.736 62.484) (end 173.736 62.484) (width 0.25) (layer F.Cu) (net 32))
 (via (at 173.736 62.484) (size 0.8) (drill 0.4) (layers F.Cu B.Cu) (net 32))
 (via (at 154.431999 64.008001) (size 0.8) (drill 0.4) (layers F.Cu B.Cu) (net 32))
 (segment (start 173.736 62.484) (end 155.956 62.484) (width 0.25) (layer B.Cu) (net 32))
 (segment (start 155.956 62.484) (end 154.431999 64.008001) (width 0.25) (layer B.Cu) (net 32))
 (segment (start 154.432 64.008) (end 154.431999 64.008001) (width 0.25) (layer F.Cu) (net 32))
 (segment (start 177.038 69.498) (end 177.038 71.628) (width 0.25) (layer F.Cu) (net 30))
 (segment (start 177.038 71.628) (end 177.038 71.628) (width 0.25) (layer F.Cu) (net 30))
 (via (at 177.038 71.628) (size 0.8) (drill 0.4) (layers F.Cu B.Cu) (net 30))
 (segment (start 181.102 78.994) (end 186.182 78.994) (width 0.25) (layer B.Cu) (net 30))
 (segment (start 177.038 74.93) (end 181.102 78.994) (width 0.25) (layer B.Cu) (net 30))
 (segment (start 186.182 78.994) (end 188.468 81.28) (width 0.25) (layer B.Cu) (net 30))
 (segment (start 177.038 71.628) (end 177.038 74.93) (width 0.25) (layer B.Cu) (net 30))
 (segment (start 180.848 69.498) (end 180.848 71.628) (width 0.25) (layer F.Cu) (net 31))
 (segment (start 180.848 71.628) (end 180.848 71.628) (width 0.25) (layer F.Cu) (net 31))
 (via (at 180.848 71.628) (size 0.8) (drill 0.4) (layers F.Cu B.Cu) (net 31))
 (segment (start 187.96 78.232) (end 191.008 81.28) (width 0.25) (layer B.Cu) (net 31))
 (segment (start 184.404 78.232) (end 187.96 78.232) (width 0.25) (layer B.Cu) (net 31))
 (segment (start 182.118 75.946) (end 184.404 78.232) (width 0.25) (layer B.Cu) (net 31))
 (segment (start 182.118 72.898) (end 182.118 75.946) (width 0.25) (layer B.Cu) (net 31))
 (segment (start 180.848 71.628) (end 182.118 72.898) (width 0.25) (layer B.Cu) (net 31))
 (segment (start 178.308 57.1135) (end 178.3445 57.15) (width 0.25) (layer F.Cu) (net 2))
 (segment (start 178.308 53.721) (end 178.308 57.1135) (width 0.25) (layer F.Cu) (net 2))
 (segment (start 178.3445 60.1615) (end 178.308 60.198) (width 0.25) (layer F.Cu) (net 2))
 (segment (start 178.3445 57.15) (end 178.3445 60.1615) (width 0.25) (layer F.Cu) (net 2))
 (segment (start 161.5805 82.7675) (end 163.068 81.28) (width 0.25) (layer F.Cu) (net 2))
 (segment (start 155.448 82.7675) (end 161.5805 82.7675) (width 0.25) (layer F.Cu) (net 2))
 (segment (start 202.692 59.944) (end 194.564 51.816) (width 0.25) (layer B.Cu) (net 2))
 (segment (start 202.692 78.041706) (end 202.692 59.944) (width 0.25) (layer B.Cu) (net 2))
 (segment (start 194.564 51.816) (end 180.213 51.816) (width 0.25) (layer B.Cu) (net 2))
 (segment (start 195.643706 85.09) (end 202.692 78.041706) (width 0.25) (layer B.Cu) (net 2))
 (segment (start 166.878 85.09) (end 195.643706 85.09) (width 0.25) (layer B.Cu) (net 2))
 (segment (start 180.213 51.816) (end 178.308 53.721) (width 0.25) (layer B.Cu) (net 2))
 (segment (start 163.068 81.28) (end 166.878 85.09) (width 0.25) (layer B.Cu) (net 2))
 (segment (start 175.768 57.1135) (end 175.7315 57.15) (width 0.25) (layer F.Cu) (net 3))
 (segment (start 175.768 53.721) (end 175.768 57.1135) (width 0.25) (layer F.Cu) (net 3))
 (segment (start 175.7315 58.8915) (end 177.038 60.198) (width 0.25) (layer F.Cu) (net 3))
 (segment (start 175.7315 57.15) (end 175.7315 58.8915) (width 0.25) (layer F.Cu) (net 3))
 (segment (start 152.9445 84.074) (end 165.354 84.074) (width 0.25) (layer F.Cu) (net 3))
 (segment (start 165.354 84.074) (end 168.148 81.28) (width 0.25) (layer F.Cu) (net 3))
 (segment (start 151.638 82.7675) (end 152.9445 84.074) (width 0.25) (layer F.Cu) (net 3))
 (segment (start 192.278 57.912) (end 179.959 57.912) (width 0.25) (layer B.Cu) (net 3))
 (segment (start 201.93 67.564) (end 192.278 57.912) (width 0.25) (layer B.Cu) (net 3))
 (segment (start 201.93 77.723002) (end 201.93 67.564) (width 0.25) (layer B.Cu) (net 3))
 (segment (start 179.959 57.912) (end 175.768 53.721) (width 0.25) (layer B.Cu) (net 3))
 (segment (start 195.325002 84.328) (end 201.93 77.723002) (width 0.25) (layer B.Cu) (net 3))
 (segment (start 171.196 84.328) (end 195.325002 84.328) (width 0.25) (layer B.Cu) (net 3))
 (segment (start 168.148 81.28) (end 171.196 84.328) (width 0.25) (layer B.Cu) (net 3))
 (segment (start 144.78 80.264) (end 154.94 70.104) (width 0.25) (layer F.Cu) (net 6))
 (segment (start 144.78 81.026) (end 144.78 80.264) (width 0.25) (layer F.Cu) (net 6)))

